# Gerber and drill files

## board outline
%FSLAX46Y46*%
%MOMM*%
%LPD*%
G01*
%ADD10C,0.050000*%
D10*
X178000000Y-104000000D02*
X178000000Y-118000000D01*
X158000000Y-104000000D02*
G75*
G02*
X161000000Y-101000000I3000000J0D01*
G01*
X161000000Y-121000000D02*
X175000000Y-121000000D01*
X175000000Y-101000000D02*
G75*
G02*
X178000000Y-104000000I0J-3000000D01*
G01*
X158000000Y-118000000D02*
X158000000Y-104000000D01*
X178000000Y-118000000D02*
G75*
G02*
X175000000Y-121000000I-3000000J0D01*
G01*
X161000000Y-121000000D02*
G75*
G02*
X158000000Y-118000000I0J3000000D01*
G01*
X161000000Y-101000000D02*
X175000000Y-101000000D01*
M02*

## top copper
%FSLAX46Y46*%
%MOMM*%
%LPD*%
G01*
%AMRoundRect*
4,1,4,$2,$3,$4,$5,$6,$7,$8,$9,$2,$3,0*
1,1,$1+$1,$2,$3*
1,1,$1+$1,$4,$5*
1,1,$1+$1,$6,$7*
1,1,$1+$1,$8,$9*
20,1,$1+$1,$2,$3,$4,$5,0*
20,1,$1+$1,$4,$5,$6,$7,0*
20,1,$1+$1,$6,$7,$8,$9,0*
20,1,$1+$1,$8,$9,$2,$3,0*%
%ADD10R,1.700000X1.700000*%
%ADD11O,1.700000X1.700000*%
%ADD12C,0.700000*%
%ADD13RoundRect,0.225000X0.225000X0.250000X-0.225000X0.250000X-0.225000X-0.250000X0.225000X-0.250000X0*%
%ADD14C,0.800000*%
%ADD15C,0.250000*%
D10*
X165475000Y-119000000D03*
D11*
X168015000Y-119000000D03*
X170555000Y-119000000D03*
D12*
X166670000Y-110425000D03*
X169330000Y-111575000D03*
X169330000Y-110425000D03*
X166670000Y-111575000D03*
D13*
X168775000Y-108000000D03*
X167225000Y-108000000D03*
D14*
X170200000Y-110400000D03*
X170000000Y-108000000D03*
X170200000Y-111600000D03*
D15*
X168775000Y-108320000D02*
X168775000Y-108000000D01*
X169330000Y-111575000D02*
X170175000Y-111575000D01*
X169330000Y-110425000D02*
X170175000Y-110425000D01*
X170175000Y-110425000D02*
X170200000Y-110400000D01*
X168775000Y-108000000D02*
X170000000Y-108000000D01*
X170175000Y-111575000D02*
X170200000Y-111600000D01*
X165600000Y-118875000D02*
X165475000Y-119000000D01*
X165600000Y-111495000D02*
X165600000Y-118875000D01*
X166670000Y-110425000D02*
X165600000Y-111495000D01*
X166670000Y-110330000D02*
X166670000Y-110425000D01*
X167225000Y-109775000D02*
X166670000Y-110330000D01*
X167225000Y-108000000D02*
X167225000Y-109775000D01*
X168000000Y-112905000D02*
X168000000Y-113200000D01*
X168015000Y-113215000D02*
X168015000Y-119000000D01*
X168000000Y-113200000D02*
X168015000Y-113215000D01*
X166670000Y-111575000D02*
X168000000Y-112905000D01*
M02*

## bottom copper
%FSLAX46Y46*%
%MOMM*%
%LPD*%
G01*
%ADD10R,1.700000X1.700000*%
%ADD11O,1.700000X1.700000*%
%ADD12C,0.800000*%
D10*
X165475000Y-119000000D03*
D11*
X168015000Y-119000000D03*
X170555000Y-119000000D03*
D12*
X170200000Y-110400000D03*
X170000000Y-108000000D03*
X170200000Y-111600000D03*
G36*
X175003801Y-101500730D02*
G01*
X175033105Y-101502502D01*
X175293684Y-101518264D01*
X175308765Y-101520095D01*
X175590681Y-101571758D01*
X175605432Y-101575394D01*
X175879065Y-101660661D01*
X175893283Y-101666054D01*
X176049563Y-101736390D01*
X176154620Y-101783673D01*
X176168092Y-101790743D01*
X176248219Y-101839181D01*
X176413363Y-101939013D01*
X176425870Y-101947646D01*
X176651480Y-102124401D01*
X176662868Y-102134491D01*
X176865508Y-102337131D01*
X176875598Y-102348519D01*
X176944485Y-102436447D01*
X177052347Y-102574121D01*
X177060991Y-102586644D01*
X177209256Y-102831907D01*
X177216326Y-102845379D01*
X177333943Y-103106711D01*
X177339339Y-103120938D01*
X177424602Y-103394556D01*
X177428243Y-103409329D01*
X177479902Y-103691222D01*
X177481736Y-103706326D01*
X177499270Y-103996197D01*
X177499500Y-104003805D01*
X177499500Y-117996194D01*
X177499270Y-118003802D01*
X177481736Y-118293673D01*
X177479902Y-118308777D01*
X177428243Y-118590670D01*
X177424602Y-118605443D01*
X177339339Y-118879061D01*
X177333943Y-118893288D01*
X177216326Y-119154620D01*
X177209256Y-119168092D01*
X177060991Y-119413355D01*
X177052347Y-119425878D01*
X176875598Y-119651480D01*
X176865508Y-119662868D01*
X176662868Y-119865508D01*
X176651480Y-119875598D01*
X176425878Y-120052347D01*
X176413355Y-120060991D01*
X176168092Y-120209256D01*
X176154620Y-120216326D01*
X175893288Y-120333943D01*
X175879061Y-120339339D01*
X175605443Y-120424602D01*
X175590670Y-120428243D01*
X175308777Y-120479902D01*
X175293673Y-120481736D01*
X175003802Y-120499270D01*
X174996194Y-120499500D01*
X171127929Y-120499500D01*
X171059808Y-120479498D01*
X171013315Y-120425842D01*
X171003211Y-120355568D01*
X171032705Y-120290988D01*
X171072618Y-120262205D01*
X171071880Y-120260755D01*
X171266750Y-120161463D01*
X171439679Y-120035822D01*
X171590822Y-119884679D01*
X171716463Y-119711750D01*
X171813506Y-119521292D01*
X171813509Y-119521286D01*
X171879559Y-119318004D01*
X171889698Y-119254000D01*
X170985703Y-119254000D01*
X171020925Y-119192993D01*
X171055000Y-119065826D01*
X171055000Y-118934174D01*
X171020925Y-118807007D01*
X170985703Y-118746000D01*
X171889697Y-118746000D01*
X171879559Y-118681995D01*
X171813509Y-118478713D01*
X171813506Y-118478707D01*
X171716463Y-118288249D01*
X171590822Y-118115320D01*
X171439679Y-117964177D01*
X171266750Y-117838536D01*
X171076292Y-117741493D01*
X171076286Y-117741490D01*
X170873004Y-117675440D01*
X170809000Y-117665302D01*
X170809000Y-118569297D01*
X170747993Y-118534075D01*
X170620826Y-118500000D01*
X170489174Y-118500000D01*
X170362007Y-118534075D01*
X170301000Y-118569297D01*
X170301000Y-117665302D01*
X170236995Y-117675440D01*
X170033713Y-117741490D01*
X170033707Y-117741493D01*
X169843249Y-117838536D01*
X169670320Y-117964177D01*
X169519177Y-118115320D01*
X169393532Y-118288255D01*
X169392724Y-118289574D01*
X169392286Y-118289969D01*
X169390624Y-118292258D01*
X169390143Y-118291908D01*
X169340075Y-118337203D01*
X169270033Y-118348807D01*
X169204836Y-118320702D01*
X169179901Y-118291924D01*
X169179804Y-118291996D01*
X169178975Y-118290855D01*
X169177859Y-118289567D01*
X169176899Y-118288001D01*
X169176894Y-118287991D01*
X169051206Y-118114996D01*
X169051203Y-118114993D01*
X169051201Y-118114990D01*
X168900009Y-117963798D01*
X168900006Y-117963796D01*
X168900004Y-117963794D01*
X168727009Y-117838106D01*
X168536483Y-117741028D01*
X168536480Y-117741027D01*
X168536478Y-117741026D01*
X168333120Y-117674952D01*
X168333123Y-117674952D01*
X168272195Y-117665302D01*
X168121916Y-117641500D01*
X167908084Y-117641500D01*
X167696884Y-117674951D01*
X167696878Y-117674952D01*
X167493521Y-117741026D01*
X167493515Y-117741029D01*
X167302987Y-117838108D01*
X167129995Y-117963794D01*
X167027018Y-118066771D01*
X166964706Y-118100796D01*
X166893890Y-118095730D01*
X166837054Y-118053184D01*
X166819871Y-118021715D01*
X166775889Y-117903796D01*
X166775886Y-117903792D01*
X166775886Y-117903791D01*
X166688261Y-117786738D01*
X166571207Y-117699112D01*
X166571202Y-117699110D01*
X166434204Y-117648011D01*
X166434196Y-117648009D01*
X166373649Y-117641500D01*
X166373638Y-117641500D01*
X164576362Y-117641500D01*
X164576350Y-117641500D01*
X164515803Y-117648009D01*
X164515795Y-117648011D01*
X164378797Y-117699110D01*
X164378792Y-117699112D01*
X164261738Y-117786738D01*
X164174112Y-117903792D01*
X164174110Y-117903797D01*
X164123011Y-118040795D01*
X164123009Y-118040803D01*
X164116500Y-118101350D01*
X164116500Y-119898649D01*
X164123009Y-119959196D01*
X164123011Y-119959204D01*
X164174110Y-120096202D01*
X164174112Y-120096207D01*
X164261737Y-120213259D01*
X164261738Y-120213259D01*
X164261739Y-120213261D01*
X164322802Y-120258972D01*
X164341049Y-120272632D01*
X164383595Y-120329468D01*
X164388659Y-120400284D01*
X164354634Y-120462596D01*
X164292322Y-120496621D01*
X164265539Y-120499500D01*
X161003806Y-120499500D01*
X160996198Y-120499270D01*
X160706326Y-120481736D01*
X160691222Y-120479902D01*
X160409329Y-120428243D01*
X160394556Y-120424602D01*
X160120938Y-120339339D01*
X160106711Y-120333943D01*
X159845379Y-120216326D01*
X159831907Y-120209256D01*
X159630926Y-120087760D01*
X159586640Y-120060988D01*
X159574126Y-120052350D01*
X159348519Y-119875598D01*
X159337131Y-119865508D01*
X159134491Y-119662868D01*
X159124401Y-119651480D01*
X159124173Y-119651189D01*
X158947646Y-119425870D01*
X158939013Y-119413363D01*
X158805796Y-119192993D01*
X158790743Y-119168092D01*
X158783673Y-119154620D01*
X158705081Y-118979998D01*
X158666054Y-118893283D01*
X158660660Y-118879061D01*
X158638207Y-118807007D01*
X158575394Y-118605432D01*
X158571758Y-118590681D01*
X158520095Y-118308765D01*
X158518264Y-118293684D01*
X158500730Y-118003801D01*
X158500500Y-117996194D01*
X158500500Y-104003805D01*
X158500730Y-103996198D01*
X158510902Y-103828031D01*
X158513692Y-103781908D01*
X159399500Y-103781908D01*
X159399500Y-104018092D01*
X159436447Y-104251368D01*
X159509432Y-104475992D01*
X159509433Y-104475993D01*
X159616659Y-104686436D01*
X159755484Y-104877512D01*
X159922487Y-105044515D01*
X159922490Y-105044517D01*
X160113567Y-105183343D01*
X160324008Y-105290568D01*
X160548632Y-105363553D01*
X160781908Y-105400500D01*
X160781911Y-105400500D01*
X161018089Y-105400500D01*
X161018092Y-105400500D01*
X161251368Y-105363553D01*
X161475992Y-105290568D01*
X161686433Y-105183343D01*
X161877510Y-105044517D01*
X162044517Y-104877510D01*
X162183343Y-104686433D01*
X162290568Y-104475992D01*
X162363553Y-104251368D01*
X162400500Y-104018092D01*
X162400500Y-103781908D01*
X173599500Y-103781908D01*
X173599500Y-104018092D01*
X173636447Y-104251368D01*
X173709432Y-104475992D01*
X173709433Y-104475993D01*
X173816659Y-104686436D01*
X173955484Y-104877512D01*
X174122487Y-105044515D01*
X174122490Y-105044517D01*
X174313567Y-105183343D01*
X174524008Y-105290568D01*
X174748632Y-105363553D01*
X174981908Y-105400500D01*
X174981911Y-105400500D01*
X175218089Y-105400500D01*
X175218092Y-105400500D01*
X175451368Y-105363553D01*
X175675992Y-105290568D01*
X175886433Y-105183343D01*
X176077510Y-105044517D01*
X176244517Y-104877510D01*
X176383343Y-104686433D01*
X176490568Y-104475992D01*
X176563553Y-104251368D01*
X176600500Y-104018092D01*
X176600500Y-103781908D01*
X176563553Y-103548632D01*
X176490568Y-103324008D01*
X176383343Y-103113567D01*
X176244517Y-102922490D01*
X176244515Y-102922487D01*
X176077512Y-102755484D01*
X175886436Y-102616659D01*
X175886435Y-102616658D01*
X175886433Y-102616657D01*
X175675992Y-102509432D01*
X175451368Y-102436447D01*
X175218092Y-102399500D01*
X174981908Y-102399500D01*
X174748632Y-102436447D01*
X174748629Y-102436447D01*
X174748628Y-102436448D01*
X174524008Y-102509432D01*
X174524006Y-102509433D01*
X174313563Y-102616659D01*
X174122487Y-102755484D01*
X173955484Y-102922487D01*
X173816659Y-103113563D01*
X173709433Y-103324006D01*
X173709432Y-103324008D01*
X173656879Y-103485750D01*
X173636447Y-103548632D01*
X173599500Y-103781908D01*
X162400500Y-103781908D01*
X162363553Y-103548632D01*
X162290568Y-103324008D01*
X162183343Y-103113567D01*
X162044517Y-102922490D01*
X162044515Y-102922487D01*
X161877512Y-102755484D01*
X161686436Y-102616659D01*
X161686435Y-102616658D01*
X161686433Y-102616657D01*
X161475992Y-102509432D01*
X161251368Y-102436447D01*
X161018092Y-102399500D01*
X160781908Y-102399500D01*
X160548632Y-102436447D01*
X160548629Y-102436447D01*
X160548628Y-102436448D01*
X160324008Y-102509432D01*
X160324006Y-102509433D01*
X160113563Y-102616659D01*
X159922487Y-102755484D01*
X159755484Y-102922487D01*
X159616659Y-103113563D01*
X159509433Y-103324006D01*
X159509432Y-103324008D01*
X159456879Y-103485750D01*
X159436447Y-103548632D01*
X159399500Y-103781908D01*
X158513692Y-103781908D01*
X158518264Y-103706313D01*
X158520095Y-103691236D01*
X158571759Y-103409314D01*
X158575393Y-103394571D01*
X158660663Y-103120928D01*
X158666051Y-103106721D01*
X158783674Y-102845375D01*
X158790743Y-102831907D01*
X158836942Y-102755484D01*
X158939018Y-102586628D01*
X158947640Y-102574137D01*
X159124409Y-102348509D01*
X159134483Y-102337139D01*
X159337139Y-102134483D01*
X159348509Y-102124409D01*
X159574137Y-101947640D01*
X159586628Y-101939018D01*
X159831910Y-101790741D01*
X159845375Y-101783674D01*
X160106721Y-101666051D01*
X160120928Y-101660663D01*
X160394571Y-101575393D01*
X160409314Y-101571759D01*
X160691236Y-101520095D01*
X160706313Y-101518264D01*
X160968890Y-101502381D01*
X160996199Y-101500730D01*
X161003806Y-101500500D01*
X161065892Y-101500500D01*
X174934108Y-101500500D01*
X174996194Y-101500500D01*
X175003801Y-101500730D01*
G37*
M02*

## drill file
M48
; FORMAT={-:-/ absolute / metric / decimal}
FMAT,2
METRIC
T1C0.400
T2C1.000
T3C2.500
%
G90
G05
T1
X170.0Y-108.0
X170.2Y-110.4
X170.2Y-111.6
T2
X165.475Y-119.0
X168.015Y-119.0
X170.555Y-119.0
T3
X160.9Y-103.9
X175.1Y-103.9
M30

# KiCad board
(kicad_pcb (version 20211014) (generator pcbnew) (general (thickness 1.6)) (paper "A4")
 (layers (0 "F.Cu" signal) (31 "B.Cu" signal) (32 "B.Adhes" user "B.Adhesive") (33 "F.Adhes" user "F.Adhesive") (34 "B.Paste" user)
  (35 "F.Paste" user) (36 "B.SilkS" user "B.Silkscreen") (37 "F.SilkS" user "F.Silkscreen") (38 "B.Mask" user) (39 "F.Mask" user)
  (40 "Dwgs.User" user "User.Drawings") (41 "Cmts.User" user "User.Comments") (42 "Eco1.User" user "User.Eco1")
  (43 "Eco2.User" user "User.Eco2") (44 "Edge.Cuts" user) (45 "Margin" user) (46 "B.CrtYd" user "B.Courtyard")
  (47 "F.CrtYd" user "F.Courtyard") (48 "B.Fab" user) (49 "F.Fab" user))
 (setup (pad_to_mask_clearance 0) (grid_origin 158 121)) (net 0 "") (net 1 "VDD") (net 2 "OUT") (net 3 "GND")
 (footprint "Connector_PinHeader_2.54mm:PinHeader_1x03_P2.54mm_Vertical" (layer "F.Cu") (at 165.475 119 90)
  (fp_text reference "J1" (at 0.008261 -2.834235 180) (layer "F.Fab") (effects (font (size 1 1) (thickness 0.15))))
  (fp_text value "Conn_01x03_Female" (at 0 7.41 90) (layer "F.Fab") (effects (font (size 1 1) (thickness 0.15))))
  (pad "1" thru_hole rect locked (at 0 0 90) (size 1.7 1.7) (drill 1) (layers *.Cu *.Mask) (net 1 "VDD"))
  (pad "2" thru_hole oval locked (at 0 2.54 90) (size 1.7 1.7) (drill 1) (layers *.Cu *.Mask) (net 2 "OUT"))
  (pad "3" thru_hole oval locked (at 0 5.08 90) (size 1.7 1.7) (drill 1) (layers *.Cu *.Mask) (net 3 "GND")))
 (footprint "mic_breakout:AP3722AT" (layer "F.Cu") (at 168 111 90)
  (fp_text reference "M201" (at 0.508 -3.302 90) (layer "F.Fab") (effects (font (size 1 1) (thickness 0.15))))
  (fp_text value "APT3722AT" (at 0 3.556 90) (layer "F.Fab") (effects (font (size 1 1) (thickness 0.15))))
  (pad "1" smd circle locked (at 0.575 -1.33 90) (size 0.7 0.7) (layers "F.Cu" "F.Paste" "F.Mask") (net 1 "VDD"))
  (pad "2" smd circle locked (at -0.575 1.33 90) (size 0.7 0.7) (layers "F.Cu" "F.Paste" "F.Mask") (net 3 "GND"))
  (pad "2" smd circle locked (at 0.575 1.33 90) (size 0.7 0.7) (layers "F.Cu" "F.Paste" "F.Mask") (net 3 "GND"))
  (pad "3" smd circle locked (at -0.575 -1.33 90) (size 0.7 0.7) (layers "F.Cu" "F.Paste" "F.Mask") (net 2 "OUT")))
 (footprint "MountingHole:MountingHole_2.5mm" (layer "F.Cu") (at 160.9 103.9)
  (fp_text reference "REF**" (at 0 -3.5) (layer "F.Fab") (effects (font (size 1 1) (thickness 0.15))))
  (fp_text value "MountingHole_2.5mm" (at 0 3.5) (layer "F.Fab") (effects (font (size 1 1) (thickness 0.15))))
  (pad "" np_thru_hole circle locked (at 0 0) (size 2.5 2.5) (drill 2.5) (layers *.Cu *.Mask)))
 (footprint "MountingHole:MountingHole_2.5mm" (layer "F.Cu") (at 175.1 103.9)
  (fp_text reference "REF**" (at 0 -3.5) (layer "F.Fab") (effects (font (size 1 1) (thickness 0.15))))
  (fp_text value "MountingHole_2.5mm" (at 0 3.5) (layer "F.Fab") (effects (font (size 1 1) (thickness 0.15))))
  (pad "" np_thru_hole circle locked (at 0 0) (size 2.5 2.5) (drill 2.5) (layers *.Cu *.Mask)))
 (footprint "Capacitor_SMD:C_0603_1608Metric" (layer "F.Cu") (at 168 108 180)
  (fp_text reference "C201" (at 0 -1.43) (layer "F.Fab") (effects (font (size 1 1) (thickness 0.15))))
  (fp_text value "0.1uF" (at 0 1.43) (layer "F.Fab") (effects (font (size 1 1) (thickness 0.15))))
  (pad "1" smd roundrect locked (at -0.775 0 180) (size 0.9 0.95) (layers "F.Cu" "F.Paste" "F.Mask") (roundrect_rratio 0.25) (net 3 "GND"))
  (pad "2" smd roundrect locked (at 0.775 0 180) (size 0.9 0.95) (layers "F.Cu" "F.Paste" "F.Mask") (roundrect_rratio 0.25) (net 1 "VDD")))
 (gr_line (start 178 104) (end 178 118) (layer "Edge.Cuts") (width 0.05))
 (gr_arc (start 158 104) (mid 158.87868 101.87868) (end 161 101) (layer "Edge.Cuts") (width 0.05))
 (gr_line (start 161 121) (end 175 121) (layer "Edge.Cuts") (width 0.05))
 (gr_arc (start 175 101) (mid 177.12132 101.87868) (end 178 104) (layer "Edge.Cuts") (width 0.05))
 (gr_line (start 158 118) (end 158 104) (layer "Edge.Cuts") (width 0.05))
 (gr_arc (start 178 118) (mid 177.12132 120.12132) (end 175 121) (layer "Edge.Cuts") (width 0.05))
 (gr_arc (start 161 121) (mid 158.87868 120.12132) (end 158 118) (layer "Edge.Cuts") (width 0.05))
 (gr_line (start 161 101) (end 175 101) (layer "Edge.Cuts") (width 0.05))
 (segment (start 168.775 108.32) (end 168.775 108) (width 0.25) (layer "F.Cu") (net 3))
 (segment (start 169.33 111.575) (end 170.175 111.575) (width 0.25) (layer "F.Cu") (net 3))
 (segment (start 169.33 110.425) (end 170.175 110.425) (width 0.25) (layer "F.Cu") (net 3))
 (segment (start 170.175 110.425) (end 170.2 110.4) (width 0.25) (layer "F.Cu") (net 3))
 (segment (start 168.775 108) (end 170 108) (width 0.25) (layer "F.Cu") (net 3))
 (segment (start 170.175 111.575) (end 170.2 111.6) (width 0.25) (layer "F.Cu") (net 3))
 (via (at 170.2 110.4) (size 0.8) (drill 0.4) (layers "F.Cu" "B.Cu") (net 3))
 (via (at 170 108) (size 0.8) (drill 0.4) (layers "F.Cu" "B.Cu") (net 3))
 (via (at 170.2 111.6) (size 0.8) (drill 0.4) (layers "F.Cu" "B.Cu") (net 3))
 (segment (start 165.6 118.875) (end 165.475 119) (width 0.25) (layer "F.Cu") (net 1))
 (segment (start 165.6 111.495) (end 165.6 118.875) (width 0.25) (layer "F.Cu") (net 1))
 (segment (start 166.67 110.425) (end 165.6 111.495) (width 0.25) (layer "F.Cu") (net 1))
 (segment (start 166.67 110.33) (end 166.67 110.425) (width 0.25) (layer "F.Cu") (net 1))
 (segment (start 167.225 109.775) (end 166.67 110.33) (width 0.25) (layer "F.Cu") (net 1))
 (segment (start 167.225 108) (end 167.225 109.775) (width 0.25) (layer "F.Cu") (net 1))
 (segment (start 168 112.905) (end 168 113.2) (width 0.25) (layer "F.Cu") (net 2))
 (segment (start 168.015 113.215) (end 168.015 119) (width 0.25) (layer "F.Cu") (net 2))
 (segment (start 168 113.2) (end 168.015 113.215) (width 0.25) (layer "F.Cu") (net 2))
 (segment (start 166.67 111.575) (end 168 112.905) (width 0.25) (layer "F.Cu") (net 2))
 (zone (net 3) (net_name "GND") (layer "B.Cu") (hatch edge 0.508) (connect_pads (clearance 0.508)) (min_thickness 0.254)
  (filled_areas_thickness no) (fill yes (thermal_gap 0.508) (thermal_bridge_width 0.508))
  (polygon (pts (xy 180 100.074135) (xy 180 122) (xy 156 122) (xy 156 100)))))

